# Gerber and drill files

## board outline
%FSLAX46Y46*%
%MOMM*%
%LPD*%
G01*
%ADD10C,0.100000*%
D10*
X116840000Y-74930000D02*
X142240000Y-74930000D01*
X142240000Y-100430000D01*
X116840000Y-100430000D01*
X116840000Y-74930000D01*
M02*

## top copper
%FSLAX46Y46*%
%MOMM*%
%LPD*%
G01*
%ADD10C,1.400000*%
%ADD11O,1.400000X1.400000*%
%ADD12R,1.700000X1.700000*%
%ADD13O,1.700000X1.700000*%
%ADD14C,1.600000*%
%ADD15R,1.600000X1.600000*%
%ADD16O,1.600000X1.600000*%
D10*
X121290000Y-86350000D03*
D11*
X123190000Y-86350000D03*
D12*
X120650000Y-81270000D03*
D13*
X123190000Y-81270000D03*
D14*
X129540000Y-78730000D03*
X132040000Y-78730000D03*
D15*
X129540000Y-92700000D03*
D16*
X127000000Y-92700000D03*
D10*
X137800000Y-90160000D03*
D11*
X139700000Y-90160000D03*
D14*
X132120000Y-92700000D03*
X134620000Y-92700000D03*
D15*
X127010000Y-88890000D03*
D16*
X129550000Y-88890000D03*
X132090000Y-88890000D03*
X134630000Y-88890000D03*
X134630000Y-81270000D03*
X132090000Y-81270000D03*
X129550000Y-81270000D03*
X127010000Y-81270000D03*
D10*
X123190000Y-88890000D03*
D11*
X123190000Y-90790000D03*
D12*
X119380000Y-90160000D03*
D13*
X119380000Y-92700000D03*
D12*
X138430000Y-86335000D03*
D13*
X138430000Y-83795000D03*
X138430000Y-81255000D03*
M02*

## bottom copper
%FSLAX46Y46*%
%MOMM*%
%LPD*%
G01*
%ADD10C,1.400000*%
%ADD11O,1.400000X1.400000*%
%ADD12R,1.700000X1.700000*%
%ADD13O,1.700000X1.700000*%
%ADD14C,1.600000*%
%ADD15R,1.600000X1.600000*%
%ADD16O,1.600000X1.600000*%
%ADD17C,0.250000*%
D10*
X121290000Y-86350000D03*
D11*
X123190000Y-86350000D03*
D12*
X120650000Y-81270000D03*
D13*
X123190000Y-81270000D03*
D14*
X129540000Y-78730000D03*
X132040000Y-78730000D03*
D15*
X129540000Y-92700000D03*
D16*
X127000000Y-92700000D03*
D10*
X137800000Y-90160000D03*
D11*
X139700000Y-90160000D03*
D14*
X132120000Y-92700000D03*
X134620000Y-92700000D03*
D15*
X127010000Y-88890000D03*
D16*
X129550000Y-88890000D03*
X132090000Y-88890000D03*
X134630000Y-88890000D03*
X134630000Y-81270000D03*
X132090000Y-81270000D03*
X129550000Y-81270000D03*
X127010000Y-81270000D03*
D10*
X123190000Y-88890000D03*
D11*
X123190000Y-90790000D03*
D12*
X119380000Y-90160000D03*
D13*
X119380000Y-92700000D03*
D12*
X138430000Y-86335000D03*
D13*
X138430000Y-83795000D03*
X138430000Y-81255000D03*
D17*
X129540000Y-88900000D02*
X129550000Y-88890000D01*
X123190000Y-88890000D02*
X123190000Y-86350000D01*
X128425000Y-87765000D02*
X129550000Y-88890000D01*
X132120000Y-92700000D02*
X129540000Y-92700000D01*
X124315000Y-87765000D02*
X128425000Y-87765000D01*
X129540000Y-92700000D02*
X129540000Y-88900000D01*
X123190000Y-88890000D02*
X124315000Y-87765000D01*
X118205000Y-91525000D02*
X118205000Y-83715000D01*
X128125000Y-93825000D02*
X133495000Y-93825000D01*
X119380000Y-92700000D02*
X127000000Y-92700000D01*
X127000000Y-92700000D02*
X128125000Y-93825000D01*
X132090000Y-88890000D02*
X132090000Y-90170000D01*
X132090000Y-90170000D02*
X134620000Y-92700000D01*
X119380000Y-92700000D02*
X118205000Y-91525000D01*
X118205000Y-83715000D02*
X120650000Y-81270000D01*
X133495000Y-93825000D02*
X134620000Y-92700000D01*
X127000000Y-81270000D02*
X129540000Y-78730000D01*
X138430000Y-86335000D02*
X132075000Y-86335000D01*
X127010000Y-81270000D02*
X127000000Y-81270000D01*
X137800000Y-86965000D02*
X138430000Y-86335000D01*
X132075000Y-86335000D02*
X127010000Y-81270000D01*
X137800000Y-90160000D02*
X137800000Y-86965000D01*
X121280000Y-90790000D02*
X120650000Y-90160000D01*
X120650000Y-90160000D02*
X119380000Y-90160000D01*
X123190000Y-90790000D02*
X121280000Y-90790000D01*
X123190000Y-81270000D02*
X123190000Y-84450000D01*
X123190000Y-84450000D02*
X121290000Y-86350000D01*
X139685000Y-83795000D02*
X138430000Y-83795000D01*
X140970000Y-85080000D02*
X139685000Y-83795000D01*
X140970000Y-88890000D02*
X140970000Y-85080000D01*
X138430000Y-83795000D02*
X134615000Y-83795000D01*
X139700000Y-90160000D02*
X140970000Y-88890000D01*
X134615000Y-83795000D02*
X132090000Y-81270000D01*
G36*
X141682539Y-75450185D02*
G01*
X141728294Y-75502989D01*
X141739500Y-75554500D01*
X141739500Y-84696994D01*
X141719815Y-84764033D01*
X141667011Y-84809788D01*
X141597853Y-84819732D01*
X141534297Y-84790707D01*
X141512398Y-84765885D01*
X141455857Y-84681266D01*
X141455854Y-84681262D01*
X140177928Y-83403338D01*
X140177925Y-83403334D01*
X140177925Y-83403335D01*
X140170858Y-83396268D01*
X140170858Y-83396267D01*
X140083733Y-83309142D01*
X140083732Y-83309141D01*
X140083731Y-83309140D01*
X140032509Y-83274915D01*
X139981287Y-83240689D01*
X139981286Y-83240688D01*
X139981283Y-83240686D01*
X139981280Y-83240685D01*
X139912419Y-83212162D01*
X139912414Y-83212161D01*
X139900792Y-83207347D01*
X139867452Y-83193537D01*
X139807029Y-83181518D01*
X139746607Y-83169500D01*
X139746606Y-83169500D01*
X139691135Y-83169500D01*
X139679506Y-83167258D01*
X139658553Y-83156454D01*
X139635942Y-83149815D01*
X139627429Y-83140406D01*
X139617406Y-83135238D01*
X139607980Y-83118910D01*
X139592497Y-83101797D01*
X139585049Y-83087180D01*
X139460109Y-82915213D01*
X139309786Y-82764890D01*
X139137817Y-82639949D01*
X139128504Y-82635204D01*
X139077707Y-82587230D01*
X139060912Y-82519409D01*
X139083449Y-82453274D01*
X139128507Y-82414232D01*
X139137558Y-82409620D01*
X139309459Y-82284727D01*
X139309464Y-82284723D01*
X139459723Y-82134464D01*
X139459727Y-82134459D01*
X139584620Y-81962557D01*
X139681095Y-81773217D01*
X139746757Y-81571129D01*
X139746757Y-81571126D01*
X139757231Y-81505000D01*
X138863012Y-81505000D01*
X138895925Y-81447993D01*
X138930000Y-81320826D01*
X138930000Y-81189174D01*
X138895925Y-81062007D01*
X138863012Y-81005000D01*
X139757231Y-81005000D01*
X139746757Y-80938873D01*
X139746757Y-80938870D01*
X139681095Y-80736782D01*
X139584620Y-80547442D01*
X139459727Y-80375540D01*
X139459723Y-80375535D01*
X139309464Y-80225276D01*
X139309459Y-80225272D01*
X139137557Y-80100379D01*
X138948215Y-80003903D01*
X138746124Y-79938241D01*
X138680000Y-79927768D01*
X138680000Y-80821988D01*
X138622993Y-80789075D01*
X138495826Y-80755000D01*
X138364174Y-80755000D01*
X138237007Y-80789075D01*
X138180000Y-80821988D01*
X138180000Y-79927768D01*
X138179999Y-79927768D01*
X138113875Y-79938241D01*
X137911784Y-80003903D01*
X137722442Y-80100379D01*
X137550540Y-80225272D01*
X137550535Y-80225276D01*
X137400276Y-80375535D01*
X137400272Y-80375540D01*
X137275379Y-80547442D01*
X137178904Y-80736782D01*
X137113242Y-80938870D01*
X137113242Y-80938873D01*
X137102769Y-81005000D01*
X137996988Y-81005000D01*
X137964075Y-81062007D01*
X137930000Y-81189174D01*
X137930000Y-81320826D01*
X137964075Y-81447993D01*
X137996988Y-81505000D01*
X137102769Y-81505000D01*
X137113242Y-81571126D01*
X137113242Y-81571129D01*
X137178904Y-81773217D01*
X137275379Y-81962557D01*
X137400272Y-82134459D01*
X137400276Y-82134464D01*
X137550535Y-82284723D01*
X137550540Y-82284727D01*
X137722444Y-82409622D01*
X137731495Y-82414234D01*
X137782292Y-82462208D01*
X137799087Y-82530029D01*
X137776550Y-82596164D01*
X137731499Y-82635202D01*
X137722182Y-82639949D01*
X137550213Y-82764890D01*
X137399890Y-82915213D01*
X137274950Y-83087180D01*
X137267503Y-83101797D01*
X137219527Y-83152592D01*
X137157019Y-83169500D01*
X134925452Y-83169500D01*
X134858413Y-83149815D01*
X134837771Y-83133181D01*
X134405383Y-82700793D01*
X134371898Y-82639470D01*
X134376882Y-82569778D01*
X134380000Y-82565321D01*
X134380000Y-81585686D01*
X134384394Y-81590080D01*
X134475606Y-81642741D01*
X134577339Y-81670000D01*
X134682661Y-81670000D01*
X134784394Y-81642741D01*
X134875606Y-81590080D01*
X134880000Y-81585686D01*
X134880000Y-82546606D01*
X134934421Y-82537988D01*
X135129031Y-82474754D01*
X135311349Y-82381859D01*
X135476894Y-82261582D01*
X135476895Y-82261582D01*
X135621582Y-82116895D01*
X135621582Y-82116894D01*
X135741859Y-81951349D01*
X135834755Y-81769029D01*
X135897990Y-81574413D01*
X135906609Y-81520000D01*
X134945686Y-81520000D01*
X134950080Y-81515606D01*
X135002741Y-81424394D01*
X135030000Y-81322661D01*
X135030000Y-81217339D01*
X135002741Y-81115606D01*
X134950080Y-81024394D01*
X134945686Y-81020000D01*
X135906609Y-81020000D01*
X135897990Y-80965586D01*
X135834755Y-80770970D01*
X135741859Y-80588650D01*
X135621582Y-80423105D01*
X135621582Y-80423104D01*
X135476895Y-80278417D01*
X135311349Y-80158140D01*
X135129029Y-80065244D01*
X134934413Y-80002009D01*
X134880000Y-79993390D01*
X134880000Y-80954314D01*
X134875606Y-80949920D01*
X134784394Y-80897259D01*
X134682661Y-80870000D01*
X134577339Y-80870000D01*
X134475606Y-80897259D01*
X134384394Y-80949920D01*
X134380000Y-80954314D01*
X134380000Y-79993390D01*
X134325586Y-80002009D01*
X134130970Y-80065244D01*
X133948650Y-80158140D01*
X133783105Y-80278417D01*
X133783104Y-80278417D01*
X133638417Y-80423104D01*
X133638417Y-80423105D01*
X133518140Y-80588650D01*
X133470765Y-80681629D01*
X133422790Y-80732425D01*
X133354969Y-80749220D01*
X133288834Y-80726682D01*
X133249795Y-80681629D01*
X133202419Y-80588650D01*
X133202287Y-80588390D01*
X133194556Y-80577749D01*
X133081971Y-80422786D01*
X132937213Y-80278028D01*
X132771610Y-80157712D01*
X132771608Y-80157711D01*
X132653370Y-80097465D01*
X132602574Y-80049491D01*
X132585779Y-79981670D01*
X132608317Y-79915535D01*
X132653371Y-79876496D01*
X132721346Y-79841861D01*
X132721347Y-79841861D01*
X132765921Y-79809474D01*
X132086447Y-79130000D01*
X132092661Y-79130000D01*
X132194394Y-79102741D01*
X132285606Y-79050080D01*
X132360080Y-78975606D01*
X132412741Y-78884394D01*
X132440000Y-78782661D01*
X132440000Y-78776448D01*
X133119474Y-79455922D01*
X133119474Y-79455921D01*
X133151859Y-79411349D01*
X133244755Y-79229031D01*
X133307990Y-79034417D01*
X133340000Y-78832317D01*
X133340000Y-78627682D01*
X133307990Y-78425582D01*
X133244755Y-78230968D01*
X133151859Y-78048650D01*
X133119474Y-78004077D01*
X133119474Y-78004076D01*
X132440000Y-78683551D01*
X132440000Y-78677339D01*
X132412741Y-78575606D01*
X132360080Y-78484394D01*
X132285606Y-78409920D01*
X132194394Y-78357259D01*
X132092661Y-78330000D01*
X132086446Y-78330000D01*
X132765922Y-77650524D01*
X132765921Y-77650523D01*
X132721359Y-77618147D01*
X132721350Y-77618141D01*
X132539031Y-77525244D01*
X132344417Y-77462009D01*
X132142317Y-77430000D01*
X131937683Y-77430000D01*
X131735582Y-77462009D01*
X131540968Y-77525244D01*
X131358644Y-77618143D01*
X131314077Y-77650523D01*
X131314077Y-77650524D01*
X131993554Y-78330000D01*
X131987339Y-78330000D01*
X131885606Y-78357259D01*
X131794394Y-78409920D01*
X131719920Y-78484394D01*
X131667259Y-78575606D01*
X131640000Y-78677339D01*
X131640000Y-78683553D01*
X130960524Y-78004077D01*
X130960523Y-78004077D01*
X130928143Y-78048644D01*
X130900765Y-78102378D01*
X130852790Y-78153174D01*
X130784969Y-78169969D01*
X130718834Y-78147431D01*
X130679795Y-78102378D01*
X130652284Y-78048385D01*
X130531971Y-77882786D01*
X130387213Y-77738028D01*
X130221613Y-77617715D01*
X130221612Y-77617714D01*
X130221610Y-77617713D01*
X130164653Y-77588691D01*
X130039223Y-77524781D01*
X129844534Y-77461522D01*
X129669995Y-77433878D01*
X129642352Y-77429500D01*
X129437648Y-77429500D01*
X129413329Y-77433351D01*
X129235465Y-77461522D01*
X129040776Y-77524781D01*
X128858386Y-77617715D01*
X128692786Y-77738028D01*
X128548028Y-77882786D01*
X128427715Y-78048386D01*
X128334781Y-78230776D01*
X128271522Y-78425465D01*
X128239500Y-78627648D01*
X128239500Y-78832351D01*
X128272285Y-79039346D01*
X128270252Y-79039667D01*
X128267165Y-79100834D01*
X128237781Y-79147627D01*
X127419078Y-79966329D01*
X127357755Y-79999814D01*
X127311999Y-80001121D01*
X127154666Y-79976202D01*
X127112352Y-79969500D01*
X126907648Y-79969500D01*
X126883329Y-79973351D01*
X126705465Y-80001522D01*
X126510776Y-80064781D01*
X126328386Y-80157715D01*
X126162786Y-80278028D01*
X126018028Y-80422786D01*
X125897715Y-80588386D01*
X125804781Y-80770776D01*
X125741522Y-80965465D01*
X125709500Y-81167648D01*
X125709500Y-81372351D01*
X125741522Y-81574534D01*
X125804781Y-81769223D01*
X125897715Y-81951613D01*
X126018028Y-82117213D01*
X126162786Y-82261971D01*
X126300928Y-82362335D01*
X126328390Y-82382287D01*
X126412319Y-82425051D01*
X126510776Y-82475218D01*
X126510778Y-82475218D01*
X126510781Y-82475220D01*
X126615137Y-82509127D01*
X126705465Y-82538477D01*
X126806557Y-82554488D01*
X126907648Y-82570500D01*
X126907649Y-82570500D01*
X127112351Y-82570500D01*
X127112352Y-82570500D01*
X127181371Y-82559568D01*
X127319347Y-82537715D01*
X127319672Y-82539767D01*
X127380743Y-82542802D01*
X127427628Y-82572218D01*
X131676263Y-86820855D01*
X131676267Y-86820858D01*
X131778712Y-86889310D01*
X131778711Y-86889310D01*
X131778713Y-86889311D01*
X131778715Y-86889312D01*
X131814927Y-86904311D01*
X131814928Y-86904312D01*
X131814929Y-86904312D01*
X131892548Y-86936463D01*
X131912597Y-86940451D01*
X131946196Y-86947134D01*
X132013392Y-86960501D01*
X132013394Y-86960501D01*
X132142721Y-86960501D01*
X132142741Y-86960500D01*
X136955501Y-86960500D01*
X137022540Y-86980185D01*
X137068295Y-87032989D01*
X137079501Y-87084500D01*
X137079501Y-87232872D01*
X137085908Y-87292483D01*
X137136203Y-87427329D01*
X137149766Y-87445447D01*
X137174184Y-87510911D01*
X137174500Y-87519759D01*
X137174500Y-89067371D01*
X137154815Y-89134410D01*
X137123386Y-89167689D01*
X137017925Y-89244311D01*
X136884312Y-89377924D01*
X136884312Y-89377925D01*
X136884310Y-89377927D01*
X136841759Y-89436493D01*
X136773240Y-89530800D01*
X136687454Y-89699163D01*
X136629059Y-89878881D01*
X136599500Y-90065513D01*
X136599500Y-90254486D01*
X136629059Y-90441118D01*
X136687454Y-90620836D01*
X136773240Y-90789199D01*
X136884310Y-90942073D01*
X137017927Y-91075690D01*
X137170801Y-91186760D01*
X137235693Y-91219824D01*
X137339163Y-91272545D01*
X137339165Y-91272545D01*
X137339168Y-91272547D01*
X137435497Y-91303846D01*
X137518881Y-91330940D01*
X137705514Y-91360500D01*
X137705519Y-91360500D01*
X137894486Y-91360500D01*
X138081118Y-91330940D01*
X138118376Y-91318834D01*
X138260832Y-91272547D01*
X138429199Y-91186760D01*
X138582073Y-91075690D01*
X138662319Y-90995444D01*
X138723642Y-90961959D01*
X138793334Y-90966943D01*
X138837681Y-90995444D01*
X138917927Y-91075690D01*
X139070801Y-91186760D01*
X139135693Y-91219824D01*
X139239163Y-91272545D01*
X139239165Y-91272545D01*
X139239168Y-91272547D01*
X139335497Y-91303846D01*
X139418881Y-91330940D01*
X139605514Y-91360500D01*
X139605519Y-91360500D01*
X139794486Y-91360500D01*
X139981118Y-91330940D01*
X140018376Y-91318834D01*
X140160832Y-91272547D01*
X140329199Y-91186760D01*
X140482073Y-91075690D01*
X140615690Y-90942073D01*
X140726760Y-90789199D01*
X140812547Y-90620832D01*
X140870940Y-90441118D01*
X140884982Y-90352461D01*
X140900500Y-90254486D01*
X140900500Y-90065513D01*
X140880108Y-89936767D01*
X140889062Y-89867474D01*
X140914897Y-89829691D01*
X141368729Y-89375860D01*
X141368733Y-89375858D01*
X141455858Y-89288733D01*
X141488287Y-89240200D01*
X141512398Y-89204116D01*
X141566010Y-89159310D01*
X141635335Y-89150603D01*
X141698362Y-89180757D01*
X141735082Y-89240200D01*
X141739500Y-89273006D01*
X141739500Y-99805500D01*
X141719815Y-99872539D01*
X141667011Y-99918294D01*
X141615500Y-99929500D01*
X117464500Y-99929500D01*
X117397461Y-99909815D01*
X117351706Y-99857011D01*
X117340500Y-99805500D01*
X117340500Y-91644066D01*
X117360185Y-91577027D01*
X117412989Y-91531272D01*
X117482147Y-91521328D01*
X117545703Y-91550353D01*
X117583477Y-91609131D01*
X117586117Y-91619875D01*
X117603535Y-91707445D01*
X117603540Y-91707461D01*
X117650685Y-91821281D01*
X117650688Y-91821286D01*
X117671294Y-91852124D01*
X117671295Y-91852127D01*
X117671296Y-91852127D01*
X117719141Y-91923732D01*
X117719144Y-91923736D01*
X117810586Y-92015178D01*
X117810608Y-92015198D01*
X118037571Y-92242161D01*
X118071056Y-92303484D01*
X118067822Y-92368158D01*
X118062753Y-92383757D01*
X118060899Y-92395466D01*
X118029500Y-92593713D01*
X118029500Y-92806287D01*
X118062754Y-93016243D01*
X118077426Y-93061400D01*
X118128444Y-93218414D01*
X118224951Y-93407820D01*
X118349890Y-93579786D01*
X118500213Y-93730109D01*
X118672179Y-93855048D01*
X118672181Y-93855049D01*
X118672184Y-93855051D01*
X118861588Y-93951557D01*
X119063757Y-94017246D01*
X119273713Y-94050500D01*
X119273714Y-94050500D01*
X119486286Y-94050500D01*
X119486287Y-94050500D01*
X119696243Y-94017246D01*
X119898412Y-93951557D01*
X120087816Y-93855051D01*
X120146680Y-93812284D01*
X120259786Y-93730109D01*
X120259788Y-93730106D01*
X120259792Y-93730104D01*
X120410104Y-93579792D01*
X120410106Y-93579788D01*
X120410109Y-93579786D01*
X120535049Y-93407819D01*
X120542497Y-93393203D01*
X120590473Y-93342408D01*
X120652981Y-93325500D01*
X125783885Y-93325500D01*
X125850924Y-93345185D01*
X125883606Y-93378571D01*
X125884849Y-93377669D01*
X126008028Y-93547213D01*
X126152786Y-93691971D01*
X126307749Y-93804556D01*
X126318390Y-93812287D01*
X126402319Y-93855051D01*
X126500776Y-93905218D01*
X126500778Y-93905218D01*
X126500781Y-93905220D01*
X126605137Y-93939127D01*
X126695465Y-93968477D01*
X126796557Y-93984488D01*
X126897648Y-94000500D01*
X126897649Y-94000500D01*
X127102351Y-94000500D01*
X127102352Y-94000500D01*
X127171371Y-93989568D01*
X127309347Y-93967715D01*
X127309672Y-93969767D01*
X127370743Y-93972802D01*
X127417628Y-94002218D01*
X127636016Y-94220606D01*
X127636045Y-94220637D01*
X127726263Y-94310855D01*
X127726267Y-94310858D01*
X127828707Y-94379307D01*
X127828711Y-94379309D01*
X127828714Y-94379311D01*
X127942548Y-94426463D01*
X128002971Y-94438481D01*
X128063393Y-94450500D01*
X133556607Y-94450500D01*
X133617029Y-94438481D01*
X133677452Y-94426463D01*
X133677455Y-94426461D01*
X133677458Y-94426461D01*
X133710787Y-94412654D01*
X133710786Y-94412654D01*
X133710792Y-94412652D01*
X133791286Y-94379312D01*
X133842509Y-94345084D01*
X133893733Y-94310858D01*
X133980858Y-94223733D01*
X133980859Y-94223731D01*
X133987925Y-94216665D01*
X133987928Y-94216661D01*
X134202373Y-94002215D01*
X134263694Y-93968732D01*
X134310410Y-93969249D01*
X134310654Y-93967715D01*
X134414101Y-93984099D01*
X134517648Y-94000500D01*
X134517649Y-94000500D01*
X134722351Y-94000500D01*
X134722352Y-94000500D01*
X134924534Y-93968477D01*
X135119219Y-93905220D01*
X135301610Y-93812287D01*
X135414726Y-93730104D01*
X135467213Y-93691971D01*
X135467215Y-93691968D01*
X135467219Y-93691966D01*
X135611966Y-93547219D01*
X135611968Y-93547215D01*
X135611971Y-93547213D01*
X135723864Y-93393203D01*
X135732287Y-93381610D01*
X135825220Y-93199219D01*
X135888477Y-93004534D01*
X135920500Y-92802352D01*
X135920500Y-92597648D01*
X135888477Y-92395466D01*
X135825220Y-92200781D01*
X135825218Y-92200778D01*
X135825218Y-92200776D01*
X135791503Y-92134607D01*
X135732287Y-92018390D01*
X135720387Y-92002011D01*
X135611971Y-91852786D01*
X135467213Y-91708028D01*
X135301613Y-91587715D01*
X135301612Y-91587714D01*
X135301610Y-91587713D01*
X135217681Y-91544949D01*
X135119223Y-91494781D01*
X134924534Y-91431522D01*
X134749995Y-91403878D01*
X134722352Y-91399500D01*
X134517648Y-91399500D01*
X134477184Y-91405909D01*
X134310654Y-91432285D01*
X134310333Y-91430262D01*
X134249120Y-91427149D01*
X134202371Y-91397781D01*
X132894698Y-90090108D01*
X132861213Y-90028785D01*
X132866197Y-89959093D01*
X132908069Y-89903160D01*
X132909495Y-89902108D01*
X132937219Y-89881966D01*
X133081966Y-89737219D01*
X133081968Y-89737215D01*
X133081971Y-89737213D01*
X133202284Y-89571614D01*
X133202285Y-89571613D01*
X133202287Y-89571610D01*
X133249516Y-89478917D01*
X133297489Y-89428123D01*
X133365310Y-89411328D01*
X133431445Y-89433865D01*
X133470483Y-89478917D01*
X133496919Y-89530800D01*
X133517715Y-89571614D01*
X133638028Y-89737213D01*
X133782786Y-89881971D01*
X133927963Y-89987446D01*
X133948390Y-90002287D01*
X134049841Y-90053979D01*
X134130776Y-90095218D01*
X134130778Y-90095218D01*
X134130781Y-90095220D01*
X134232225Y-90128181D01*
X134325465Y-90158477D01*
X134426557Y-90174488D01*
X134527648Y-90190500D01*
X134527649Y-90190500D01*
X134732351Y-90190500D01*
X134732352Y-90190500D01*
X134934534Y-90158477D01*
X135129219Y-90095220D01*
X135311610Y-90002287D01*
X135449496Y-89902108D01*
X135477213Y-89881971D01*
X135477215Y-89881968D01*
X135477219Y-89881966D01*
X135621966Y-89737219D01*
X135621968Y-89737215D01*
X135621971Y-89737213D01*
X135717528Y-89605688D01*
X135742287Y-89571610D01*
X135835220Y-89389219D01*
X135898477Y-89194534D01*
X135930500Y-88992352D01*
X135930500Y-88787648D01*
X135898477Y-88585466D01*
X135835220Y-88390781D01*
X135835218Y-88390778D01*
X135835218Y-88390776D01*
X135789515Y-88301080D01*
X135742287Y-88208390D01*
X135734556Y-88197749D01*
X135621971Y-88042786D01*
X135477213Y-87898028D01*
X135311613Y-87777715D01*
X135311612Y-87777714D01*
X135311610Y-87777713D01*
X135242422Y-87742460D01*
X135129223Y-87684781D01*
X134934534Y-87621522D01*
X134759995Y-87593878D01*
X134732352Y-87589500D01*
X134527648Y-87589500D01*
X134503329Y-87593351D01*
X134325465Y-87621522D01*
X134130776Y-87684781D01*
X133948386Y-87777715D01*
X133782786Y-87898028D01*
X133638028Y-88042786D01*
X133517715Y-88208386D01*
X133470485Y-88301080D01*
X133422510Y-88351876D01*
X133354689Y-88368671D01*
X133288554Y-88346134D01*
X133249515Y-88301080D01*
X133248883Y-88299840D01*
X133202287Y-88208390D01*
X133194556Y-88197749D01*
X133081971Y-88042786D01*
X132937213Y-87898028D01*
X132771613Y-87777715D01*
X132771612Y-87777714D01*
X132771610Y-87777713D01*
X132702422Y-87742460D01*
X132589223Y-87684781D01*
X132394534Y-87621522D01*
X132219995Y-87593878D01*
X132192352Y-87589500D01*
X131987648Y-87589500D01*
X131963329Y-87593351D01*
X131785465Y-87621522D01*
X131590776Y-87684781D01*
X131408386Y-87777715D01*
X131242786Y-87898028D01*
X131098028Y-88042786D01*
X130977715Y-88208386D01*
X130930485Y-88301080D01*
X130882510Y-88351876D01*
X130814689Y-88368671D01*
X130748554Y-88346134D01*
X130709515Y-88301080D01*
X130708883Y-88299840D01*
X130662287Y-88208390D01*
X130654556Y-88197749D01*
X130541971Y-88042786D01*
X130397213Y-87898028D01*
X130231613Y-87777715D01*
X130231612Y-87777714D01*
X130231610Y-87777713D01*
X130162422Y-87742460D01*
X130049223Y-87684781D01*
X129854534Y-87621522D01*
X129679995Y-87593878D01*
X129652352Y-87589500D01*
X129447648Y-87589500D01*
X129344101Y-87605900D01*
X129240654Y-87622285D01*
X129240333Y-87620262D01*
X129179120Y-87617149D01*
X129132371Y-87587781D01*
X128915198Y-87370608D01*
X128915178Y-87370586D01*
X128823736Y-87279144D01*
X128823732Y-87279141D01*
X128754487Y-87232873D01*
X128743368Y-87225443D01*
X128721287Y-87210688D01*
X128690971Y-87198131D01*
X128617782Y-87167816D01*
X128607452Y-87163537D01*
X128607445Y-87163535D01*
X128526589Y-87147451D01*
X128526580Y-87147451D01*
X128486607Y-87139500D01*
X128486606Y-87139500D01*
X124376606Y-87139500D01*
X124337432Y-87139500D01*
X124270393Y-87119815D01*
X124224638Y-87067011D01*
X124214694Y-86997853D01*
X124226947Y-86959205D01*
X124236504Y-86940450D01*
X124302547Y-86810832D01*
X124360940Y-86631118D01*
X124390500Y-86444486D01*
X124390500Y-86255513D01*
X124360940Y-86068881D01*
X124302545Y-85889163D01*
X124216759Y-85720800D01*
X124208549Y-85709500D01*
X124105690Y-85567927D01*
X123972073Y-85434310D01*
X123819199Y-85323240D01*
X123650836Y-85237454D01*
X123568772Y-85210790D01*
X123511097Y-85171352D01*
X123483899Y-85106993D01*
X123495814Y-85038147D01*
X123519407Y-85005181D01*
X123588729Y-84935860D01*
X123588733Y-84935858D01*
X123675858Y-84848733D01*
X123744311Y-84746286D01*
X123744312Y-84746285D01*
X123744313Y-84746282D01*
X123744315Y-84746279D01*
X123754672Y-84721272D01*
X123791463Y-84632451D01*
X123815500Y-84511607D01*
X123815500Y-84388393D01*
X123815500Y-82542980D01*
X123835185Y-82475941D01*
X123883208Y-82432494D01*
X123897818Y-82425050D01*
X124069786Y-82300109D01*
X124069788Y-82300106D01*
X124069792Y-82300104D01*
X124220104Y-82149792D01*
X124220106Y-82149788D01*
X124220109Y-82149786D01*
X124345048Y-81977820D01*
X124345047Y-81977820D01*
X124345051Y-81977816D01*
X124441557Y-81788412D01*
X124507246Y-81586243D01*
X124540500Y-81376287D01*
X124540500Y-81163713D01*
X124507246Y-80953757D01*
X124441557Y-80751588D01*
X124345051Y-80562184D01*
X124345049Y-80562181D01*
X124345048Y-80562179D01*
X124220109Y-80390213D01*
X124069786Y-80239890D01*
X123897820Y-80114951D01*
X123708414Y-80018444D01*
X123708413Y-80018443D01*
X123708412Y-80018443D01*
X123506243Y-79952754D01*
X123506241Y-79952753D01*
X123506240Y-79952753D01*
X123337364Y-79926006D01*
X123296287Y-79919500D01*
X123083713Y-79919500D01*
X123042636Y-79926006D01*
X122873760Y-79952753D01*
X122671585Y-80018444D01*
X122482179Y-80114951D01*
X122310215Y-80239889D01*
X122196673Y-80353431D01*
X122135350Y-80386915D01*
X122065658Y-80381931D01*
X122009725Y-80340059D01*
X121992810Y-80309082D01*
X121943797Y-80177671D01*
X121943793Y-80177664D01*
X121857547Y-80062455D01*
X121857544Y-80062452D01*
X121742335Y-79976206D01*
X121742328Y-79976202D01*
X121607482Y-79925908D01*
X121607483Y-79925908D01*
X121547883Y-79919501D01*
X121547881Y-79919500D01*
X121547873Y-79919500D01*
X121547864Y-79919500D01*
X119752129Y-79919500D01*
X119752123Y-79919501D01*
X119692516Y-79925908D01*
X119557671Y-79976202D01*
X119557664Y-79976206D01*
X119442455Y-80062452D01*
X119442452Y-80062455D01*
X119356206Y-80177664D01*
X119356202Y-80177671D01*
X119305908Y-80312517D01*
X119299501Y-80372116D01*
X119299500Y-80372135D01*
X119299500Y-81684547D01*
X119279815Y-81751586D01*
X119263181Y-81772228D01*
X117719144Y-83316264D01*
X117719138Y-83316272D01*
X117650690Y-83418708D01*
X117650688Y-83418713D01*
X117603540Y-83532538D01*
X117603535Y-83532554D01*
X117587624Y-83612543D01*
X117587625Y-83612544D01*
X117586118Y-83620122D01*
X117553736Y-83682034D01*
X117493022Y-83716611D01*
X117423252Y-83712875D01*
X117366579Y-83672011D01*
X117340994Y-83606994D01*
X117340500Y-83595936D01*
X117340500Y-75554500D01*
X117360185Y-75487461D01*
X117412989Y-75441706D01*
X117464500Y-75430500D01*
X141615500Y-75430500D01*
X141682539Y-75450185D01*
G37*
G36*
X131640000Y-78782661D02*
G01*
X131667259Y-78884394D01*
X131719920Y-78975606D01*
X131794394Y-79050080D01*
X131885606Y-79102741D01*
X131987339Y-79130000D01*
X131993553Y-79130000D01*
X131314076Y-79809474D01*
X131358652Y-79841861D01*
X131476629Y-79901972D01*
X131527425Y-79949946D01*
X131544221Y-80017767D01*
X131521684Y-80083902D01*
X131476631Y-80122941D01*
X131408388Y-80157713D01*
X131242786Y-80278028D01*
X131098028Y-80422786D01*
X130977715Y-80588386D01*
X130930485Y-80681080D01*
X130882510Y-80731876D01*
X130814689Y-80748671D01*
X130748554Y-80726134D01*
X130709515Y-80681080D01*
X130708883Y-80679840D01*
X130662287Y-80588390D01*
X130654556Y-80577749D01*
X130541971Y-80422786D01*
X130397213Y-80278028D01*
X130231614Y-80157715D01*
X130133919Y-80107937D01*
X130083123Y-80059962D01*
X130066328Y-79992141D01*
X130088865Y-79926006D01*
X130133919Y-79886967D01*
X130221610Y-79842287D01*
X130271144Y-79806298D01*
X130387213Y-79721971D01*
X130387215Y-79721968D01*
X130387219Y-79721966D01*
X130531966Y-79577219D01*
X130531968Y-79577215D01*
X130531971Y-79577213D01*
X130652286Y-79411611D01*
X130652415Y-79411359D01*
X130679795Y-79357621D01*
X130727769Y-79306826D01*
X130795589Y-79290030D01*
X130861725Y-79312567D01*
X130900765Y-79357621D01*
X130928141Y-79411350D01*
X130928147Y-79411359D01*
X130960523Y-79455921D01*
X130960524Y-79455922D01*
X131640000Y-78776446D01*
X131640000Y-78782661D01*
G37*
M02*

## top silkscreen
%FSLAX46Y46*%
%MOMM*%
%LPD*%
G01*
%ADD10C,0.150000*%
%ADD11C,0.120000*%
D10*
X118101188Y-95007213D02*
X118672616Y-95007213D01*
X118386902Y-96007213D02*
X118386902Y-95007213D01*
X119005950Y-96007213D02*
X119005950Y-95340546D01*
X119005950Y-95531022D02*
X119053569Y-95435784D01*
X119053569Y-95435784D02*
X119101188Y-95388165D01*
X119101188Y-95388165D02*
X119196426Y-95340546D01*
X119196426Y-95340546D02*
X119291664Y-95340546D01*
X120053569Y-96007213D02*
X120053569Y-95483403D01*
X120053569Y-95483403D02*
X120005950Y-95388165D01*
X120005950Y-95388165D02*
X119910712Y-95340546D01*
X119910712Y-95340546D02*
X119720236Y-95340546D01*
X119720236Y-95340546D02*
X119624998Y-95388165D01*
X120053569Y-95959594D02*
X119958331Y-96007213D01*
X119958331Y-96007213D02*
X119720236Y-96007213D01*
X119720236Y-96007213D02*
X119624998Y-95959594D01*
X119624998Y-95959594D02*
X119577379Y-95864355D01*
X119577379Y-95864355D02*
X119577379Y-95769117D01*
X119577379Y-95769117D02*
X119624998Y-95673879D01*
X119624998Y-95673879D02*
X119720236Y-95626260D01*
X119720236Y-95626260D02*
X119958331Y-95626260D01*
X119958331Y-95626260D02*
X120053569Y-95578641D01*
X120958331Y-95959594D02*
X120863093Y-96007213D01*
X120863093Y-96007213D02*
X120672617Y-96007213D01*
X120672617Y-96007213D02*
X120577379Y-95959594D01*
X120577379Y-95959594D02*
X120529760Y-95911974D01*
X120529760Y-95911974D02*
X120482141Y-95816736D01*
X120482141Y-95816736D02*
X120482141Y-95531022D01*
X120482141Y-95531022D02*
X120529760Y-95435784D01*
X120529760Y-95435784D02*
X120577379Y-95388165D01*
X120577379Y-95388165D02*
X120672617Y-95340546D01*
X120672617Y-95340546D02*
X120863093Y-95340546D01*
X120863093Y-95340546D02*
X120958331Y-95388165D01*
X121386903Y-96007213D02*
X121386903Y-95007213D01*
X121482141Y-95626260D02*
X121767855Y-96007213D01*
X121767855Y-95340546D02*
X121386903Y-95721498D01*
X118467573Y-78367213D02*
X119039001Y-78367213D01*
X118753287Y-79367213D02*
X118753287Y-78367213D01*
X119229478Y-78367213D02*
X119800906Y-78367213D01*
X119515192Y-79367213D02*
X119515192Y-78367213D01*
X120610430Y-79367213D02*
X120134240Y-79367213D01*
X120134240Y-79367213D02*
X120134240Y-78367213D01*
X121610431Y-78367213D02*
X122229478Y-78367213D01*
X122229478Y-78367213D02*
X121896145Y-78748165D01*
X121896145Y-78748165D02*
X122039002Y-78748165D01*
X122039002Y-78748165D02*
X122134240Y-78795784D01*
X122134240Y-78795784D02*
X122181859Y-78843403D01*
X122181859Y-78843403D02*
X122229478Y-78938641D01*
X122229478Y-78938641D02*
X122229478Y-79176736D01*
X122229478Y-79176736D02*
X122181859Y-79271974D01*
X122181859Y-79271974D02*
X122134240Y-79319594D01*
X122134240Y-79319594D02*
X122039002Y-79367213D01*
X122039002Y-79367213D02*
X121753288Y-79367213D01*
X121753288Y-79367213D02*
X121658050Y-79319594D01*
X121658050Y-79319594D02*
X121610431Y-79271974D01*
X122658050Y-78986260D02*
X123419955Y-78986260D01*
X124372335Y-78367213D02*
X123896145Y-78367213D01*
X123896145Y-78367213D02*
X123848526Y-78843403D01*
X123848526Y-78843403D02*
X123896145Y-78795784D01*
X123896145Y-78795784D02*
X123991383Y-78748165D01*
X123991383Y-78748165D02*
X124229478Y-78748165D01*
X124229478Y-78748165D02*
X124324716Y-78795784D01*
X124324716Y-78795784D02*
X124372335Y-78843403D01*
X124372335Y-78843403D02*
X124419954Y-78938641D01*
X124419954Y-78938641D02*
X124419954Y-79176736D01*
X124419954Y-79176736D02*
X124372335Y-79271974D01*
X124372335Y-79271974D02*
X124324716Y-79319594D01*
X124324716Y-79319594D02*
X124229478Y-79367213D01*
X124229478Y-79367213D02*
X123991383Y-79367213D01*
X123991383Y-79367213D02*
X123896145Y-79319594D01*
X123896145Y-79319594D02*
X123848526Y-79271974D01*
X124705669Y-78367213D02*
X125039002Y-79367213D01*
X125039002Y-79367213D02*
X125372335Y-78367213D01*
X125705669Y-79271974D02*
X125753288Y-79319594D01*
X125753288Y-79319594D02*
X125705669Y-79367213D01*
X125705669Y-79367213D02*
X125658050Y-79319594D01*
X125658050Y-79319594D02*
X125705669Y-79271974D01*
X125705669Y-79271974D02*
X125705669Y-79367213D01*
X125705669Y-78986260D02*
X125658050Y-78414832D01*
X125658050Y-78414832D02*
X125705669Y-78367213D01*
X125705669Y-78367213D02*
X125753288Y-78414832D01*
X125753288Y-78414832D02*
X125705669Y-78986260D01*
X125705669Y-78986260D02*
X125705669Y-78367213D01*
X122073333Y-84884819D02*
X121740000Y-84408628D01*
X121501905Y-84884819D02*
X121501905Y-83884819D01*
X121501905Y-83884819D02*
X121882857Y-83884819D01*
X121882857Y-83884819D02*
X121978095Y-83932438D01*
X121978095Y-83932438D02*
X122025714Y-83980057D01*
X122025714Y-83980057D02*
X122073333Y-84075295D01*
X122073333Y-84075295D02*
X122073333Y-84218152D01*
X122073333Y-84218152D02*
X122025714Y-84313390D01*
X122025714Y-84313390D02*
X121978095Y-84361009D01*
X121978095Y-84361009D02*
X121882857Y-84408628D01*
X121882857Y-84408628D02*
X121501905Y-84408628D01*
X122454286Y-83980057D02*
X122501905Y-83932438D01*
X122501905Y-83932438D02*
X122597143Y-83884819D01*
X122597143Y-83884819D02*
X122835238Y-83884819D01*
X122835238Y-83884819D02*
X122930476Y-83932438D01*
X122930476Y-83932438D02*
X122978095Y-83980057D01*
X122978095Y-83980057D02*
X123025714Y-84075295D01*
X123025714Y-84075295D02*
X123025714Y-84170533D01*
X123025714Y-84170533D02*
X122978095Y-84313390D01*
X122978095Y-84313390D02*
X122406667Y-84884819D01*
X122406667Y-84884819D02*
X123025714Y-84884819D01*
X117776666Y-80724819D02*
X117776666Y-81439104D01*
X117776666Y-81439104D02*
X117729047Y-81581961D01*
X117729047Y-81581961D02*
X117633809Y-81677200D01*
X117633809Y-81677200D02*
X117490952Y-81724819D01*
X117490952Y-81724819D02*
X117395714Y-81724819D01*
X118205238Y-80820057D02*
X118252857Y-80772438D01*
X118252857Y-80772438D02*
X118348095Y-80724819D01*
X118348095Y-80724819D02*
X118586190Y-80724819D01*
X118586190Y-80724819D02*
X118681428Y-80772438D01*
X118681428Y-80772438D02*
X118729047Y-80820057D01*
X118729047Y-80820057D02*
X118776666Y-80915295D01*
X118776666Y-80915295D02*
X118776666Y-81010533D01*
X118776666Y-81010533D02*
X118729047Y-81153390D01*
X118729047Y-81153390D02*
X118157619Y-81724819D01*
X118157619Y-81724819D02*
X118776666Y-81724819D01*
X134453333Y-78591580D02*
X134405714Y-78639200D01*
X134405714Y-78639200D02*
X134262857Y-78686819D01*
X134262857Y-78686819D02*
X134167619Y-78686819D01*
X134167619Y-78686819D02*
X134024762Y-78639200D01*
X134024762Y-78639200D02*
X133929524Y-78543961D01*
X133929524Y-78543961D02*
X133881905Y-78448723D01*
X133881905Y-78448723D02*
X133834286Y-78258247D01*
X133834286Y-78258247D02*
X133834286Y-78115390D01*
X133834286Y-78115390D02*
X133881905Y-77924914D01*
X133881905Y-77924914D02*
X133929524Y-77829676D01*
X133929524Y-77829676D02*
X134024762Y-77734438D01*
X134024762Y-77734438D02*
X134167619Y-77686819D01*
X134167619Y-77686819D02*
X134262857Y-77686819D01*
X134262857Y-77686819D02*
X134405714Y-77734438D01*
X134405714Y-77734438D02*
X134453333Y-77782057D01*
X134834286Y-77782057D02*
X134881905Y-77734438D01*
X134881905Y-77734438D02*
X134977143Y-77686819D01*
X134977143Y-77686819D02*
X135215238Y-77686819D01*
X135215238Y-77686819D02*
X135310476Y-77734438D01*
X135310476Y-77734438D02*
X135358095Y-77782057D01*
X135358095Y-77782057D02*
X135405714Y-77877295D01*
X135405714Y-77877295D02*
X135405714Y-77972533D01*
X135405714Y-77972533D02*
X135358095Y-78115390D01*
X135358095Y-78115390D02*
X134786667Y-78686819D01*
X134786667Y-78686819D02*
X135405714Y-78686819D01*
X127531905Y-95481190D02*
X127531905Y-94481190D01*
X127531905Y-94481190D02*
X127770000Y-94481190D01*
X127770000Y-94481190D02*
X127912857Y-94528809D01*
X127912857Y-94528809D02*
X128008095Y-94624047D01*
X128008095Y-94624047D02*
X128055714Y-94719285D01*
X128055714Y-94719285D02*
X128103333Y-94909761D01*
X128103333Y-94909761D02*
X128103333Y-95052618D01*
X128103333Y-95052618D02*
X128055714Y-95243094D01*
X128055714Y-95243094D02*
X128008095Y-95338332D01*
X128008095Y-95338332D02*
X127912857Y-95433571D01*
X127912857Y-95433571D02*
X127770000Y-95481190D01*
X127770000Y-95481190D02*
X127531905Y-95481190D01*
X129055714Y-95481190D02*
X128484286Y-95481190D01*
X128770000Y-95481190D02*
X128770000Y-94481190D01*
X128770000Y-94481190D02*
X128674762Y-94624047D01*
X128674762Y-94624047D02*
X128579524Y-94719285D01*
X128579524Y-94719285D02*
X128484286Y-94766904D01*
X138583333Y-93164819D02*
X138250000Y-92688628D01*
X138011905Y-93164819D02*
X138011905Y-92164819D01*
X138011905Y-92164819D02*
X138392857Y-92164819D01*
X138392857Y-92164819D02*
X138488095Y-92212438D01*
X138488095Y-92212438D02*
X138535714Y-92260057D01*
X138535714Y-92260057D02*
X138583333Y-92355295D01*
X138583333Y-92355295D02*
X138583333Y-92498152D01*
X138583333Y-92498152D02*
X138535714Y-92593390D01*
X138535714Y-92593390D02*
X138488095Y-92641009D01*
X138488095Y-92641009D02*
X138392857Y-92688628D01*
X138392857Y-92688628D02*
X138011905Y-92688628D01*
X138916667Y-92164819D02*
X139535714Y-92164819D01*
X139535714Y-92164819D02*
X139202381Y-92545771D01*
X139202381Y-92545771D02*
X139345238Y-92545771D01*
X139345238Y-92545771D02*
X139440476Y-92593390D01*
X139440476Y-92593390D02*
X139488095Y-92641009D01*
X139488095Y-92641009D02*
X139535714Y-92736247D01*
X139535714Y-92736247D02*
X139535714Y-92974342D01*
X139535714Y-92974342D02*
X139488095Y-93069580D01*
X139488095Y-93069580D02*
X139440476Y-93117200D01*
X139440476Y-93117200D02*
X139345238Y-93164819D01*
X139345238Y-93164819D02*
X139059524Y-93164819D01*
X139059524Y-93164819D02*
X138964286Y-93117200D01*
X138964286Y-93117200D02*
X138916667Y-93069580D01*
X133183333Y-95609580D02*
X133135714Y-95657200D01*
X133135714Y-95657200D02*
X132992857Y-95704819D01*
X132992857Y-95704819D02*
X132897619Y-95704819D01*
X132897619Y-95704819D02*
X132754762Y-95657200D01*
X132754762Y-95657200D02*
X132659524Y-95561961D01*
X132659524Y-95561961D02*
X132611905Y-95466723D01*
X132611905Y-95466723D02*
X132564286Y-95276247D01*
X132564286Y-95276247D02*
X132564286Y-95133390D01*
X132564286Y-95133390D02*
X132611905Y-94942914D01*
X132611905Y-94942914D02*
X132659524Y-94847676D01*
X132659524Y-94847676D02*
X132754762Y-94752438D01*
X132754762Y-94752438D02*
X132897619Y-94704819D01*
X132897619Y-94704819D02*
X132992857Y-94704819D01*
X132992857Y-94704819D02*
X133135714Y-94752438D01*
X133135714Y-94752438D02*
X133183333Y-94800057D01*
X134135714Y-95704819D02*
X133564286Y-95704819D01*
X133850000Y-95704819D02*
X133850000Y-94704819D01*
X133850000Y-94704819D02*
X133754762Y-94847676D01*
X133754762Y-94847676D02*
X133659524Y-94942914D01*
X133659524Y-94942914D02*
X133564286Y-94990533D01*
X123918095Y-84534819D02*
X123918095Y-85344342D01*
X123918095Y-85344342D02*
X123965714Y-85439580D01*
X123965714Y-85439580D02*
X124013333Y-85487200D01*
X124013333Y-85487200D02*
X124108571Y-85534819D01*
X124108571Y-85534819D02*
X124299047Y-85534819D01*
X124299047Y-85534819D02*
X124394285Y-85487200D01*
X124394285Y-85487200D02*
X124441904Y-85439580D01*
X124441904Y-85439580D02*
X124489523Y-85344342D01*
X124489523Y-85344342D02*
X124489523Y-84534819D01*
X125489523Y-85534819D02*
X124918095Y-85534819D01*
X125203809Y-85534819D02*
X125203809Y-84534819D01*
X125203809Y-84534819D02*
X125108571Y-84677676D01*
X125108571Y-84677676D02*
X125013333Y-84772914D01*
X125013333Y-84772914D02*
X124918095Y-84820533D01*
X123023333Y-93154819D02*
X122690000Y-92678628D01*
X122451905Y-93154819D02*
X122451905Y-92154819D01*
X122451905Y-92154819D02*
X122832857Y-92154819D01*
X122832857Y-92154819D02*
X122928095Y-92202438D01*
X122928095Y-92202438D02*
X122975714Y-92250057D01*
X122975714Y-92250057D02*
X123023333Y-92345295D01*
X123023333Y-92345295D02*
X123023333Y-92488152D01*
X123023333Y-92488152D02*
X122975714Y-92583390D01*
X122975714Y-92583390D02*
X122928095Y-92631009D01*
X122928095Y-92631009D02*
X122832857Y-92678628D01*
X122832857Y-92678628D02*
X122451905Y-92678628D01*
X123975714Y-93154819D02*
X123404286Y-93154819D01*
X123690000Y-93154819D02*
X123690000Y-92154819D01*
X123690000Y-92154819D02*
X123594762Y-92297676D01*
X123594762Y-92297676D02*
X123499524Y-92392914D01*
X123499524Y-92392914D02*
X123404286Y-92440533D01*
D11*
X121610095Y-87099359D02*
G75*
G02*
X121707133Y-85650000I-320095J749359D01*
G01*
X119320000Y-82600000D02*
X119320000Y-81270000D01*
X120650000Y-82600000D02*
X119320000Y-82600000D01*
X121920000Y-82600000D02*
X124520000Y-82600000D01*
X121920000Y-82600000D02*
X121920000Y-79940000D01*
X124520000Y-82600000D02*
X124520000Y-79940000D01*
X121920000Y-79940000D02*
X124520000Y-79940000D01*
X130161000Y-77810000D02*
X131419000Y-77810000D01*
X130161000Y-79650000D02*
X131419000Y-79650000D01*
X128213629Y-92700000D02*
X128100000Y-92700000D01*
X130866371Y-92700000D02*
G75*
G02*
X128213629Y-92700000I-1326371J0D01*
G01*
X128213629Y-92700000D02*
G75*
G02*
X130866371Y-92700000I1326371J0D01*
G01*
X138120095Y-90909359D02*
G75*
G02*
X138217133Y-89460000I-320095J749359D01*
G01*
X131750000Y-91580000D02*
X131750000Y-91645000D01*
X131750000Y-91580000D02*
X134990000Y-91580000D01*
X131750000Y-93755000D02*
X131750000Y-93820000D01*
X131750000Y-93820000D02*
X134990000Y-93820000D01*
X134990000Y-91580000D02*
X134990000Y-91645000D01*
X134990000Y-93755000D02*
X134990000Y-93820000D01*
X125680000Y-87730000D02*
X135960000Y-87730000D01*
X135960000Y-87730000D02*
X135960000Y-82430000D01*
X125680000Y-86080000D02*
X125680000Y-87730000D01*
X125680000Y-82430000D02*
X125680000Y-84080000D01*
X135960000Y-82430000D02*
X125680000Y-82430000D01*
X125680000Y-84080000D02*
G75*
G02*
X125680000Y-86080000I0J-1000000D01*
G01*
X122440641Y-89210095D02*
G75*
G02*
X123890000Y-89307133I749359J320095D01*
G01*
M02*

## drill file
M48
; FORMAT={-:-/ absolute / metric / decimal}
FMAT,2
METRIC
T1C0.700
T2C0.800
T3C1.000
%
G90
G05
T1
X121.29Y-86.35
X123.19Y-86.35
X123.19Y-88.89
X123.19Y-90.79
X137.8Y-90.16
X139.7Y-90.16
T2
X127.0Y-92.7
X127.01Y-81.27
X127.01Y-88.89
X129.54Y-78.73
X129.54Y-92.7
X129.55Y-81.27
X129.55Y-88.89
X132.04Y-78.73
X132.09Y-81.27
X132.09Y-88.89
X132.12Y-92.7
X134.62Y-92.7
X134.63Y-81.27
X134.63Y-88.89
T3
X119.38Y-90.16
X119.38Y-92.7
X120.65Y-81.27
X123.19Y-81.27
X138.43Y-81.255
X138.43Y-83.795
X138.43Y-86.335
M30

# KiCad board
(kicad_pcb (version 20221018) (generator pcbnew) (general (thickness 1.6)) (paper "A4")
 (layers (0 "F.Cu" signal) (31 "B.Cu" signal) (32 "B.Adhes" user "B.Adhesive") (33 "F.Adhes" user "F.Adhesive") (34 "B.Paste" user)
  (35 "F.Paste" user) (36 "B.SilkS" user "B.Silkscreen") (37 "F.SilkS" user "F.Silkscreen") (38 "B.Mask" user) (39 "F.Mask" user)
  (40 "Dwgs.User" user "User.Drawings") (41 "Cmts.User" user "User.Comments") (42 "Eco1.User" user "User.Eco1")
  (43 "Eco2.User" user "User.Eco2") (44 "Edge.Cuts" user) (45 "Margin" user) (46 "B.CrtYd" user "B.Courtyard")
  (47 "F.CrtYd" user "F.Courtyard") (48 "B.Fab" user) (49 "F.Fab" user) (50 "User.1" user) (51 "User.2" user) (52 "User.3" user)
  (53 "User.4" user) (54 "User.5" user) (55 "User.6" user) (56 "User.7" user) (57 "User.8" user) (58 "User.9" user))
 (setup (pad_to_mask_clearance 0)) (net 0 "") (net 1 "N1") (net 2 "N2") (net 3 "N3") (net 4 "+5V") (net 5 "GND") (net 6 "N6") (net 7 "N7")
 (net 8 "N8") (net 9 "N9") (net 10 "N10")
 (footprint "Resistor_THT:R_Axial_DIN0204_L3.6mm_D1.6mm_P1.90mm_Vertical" (layer "F.Cu") (at 121.29 86.35)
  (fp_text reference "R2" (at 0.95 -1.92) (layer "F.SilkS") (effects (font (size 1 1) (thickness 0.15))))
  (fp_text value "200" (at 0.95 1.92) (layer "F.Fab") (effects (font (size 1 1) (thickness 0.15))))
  (fp_arc (start 0.320095 0.749359) (mid -0.813042 -0.054435) (end 0.417133 -0.7) (stroke (width 0.12) (type solid)) (layer "F.SilkS"))
  (pad "1" thru_hole circle (at 0 0) (size 1.4 1.4) (drill 0.7) (layers "*.Cu" "*.Mask") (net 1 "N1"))
  (pad "2" thru_hole oval (at 1.9 0) (size 1.4 1.4) (drill 0.7) (layers "*.Cu" "*.Mask") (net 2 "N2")))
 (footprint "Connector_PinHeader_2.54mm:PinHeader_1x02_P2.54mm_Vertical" (layer "F.Cu") (at 120.65 81.27 90)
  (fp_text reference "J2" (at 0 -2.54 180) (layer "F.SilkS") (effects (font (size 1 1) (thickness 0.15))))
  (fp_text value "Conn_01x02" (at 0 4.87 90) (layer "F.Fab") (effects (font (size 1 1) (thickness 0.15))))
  (fp_line (start -1.33 -1.33) (end 0 -1.33) (stroke (width 0.12) (type solid)) (layer "F.SilkS"))
  (fp_line (start -1.33 0) (end -1.33 -1.33) (stroke (width 0.12) (type solid)) (layer "F.SilkS"))
  (fp_line (start -1.33 1.27) (end -1.33 3.87) (stroke (width 0.12) (type solid)) (layer "F.SilkS"))
  (fp_line (start -1.33 1.27) (end 1.33 1.27) (stroke (width 0.12) (type solid)) (layer "F.SilkS"))
  (fp_line (start -1.33 3.87) (end 1.33 3.87) (stroke (width 0.12) (type solid)) (layer "F.SilkS"))
  (fp_line (start 1.33 1.27) (end 1.33 3.87) (stroke (width 0.12) (type solid)) (layer "F.SilkS"))
  (pad "1" thru_hole rect (at 0 0 90) (size 1.7 1.7) (drill 1) (layers "*.Cu" "*.Mask") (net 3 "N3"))
  (pad "2" thru_hole oval (at 0 2.54 90) (size 1.7 1.7) (drill 1) (layers "*.Cu" "*.Mask") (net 1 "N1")))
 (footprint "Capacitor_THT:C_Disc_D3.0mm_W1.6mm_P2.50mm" (layer "F.Cu") (at 129.54 78.73)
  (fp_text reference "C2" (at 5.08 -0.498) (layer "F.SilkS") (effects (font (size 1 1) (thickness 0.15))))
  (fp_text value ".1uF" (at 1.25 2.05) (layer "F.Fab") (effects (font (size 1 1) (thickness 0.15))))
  (fp_line (start 0.621 -0.92) (end 1.879 -0.92) (stroke (width 0.12) (type solid)) (layer "F.SilkS"))
  (fp_line (start 0.621 0.92) (end 1.879 0.92) (stroke (width 0.12) (type solid)) (layer "F.SilkS"))
  (pad "1" thru_hole circle (at 0 0) (size 1.6 1.6) (drill 0.8) (layers "*.Cu" "*.Mask") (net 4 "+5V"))
  (pad "2" thru_hole circle (at 2.5 0) (size 1.6 1.6) (drill 0.8) (layers "*.Cu" "*.Mask") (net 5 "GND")))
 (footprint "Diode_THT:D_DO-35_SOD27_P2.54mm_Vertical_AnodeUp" (layer "F.Cu") (at 129.54 92.7 180)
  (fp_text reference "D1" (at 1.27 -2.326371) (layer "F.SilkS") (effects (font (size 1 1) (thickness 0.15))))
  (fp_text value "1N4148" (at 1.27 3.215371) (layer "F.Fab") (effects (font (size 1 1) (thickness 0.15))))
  (fp_line (start 1.326371 0) (end 1.44 0) (stroke (width 0.12) (type solid)) (layer "F.SilkS"))
  (fp_circle (center 0 0) (end 1.326371 0) (stroke (width 0.12) (type solid)) (fill none) (layer "F.SilkS"))
  (pad "1" thru_hole rect (at 0 0 180) (size 1.6 1.6) (drill 0.8) (layers "*.Cu" "*.Mask") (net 2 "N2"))
  (pad "2" thru_hole oval (at 2.54 0 180) (size 1.6 1.6) (drill 0.8) (layers "*.Cu" "*.Mask") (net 3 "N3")))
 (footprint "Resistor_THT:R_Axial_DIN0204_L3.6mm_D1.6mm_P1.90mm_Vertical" (layer "F.Cu") (at 137.8 90.16)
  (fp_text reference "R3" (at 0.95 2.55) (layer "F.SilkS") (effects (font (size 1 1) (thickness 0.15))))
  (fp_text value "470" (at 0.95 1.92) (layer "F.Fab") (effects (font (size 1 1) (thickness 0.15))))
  (fp_arc (start 0.320095 0.749359) (mid -0.813042 -0.054435) (end 0.417133 -0.7) (stroke (width 0.12) (type solid)) (layer "F.SilkS"))
  (pad "1" thru_hole circle (at 0 0) (size 1.4 1.4) (drill 0.7) (layers "*.Cu" "*.Mask") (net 4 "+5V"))
  (pad "2" thru_hole oval (at 1.9 0) (size 1.4 1.4) (drill 0.7) (layers "*.Cu" "*.Mask") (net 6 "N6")))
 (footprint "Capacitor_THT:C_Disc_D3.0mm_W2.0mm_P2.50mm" (layer "F.Cu") (at 132.12 92.7)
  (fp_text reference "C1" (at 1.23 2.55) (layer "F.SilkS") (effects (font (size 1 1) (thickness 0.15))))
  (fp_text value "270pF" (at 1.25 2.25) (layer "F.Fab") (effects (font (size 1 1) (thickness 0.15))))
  (fp_line (start -0.37 -1.12) (end -0.37 -1.055) (stroke (width 0.12) (type solid)) (layer "F.SilkS"))
  (fp_line (start -0.37 -1.12) (end 2.87 -1.12) (stroke (width 0.12) (type solid)) (layer "F.SilkS"))
  (fp_line (start -0.37 1.055) (end -0.37 1.12) (stroke (width 0.12) (type solid)) (layer "F.SilkS"))
  (fp_line (start -0.37 1.12) (end 2.87 1.12) (stroke (width 0.12) (type solid)) (layer "F.SilkS"))
  (fp_line (start 2.87 -1.12) (end 2.87 -1.055) (stroke (width 0.12) (type solid)) (layer "F.SilkS"))
  (fp_line (start 2.87 1.055) (end 2.87 1.12) (stroke (width 0.12) (type solid)) (layer "F.SilkS"))
  (pad "1" thru_hole circle (at 0 0) (size 1.6 1.6) (drill 0.8) (layers "*.Cu" "*.Mask") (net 2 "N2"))
  (pad "2" thru_hole circle (at 2.5 0) (size 1.6 1.6) (drill 0.8) (layers "*.Cu" "*.Mask") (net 3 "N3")))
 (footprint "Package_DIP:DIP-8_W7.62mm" (layer "F.Cu") (at 127.01 88.89 90)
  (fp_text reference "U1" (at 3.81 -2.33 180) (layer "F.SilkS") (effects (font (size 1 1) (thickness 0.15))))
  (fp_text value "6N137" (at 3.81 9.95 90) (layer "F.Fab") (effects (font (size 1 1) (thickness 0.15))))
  (fp_line (start 1.16 -1.33) (end 1.16 8.95) (stroke (width 0.12) (type solid)) (layer "F.SilkS"))
  (fp_line (start 1.16 8.95) (end 6.46 8.95) (stroke (width 0.12) (type solid)) (layer "F.SilkS"))
  (fp_line (start 2.81 -1.33) (end 1.16 -1.33) (stroke (width 0.12) (type solid)) (layer "F.SilkS"))
  (fp_line (start 6.46 -1.33) (end 4.81 -1.33) (stroke (width 0.12) (type solid)) (layer "F.SilkS"))
  (fp_line (start 6.46 8.95) (end 6.46 -1.33) (stroke (width 0.12) (type solid)) (layer "F.SilkS"))
  (fp_arc (start 4.81 -1.33) (mid 3.81 -0.33) (end 2.81 -1.33) (stroke (width 0.12) (type solid)) (layer "F.SilkS"))
  (pad "1" thru_hole rect (at 0 0 90) (size 1.6 1.6) (drill 0.8) (layers "*.Cu" "*.Mask") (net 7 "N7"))
  (pad "2" thru_hole oval (at 0 2.54 90) (size 1.6 1.6) (drill 0.8) (layers "*.Cu" "*.Mask") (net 2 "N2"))
  (pad "3" thru_hole oval (at 0 5.08 90) (size 1.6 1.6) (drill 0.8) (layers "*.Cu" "*.Mask") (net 3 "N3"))
  (pad "4" thru_hole oval (at 0 7.62 90) (size 1.6 1.6) (drill 0.8) (layers "*.Cu" "*.Mask") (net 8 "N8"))
  (pad "5" thru_hole oval (at 7.62 7.62 90) (size 1.6 1.6) (drill 0.8) (layers "*.Cu" "*.Mask") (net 5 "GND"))
  (pad "6" thru_hole oval (at 7.62 5.08 90) (size 1.6 1.6) (drill 0.8) (layers "*.Cu" "*.Mask") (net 6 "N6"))
  (pad "7" thru_hole oval (at 7.62 2.54 90) (size 1.6 1.6) (drill 0.8) (layers "*.Cu" "*.Mask") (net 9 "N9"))
  (pad "8" thru_hole oval (at 7.62 0 90) (size 1.6 1.6) (drill 0.8) (layers "*.Cu" "*.Mask") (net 4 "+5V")))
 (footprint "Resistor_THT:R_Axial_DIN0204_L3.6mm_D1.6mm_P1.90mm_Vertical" (layer "F.Cu") (at 123.19 88.89 -90)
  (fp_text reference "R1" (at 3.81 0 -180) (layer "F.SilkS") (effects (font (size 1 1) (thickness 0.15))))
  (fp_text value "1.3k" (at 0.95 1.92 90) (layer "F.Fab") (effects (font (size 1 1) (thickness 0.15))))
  (fp_arc (start 0.320095 0.749359) (mid -0.813042 -0.054435) (end 0.417133 -0.7) (stroke (width 0.12) (type solid)) (layer "F.SilkS"))
  (pad "1" thru_hole circle (at 0 0 270) (size 1.4 1.4) (drill 0.7) (layers "*.Cu" "*.Mask") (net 2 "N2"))
  (pad "2" thru_hole oval (at 1.9 0 270) (size 1.4 1.4) (drill 0.7) (layers "*.Cu" "*.Mask") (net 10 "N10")))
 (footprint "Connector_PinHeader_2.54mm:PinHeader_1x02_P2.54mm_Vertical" (layer "B.Cu") (at 119.38 90.16 180)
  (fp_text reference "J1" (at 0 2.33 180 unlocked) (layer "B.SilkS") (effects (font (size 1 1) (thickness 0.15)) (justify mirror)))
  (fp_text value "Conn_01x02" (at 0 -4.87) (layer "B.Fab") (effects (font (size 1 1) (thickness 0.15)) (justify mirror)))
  (pad "1" thru_hole rect (at 0 0 180) (size 1.7 1.7) (drill 1) (layers "*.Cu" "*.Mask") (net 10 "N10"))
  (pad "2" thru_hole oval (at 0 -2.54 180) (size 1.7 1.7) (drill 1) (layers "*.Cu" "*.Mask") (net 3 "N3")))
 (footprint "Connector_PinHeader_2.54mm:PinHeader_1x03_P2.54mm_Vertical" (layer "B.Cu") (at 138.43 86.335)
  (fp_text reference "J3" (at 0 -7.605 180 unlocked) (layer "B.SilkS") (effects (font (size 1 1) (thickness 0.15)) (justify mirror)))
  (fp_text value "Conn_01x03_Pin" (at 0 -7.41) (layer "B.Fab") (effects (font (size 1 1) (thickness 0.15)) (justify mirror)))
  (pad "1" thru_hole rect (at 0 0) (size 1.7 1.7) (drill 1) (layers "*.Cu" "*.Mask") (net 4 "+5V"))
  (pad "2" thru_hole oval (at 0 -2.54) (size 1.7 1.7) (drill 1) (layers "*.Cu" "*.Mask") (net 6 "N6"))
  (pad "3" thru_hole oval (at 0 -5.08) (size 1.7 1.7) (drill 1) (layers "*.Cu" "*.Mask") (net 5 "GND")))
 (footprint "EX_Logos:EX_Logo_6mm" (layer "B.Cu") (at 137.668 97.028)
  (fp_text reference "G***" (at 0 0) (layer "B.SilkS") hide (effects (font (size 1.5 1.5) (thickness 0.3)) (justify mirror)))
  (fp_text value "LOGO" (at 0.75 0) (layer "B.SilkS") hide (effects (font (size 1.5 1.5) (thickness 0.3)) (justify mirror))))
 (gr_rect (start 116.84 74.93) (end 142.24 100.43) (stroke (width 0.1) (type default)) (fill none) (layer "Edge.Cuts"))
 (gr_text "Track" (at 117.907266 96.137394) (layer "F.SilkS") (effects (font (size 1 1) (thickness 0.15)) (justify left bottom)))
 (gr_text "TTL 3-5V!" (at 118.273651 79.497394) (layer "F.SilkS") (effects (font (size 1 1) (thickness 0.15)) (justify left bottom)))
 (segment (start 129.54 88.9) (end 129.55 88.89) (width 0.25) (layer "B.Cu") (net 2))
 (segment (start 123.19 88.89) (end 123.19 86.35) (width 0.25) (layer "B.Cu") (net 2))
 (segment (start 128.425 87.765) (end 129.55 88.89) (width 0.25) (layer "B.Cu") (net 2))
 (segment (start 132.12 92.7) (end 129.54 92.7) (width 0.25) (layer "B.Cu") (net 2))
 (segment (start 124.315 87.765) (end 128.425 87.765) (width 0.25) (layer "B.Cu") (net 2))
 (segment (start 129.54 92.7) (end 129.54 88.9) (width 0.25) (layer "B.Cu") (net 2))
 (segment (start 123.19 88.89) (end 124.315 87.765) (width 0.25) (layer "B.Cu") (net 2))
 (segment (start 118.205 91.525) (end 118.205 83.715) (width 0.25) (layer "B.Cu") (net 3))
 (segment (start 128.125 93.825) (end 133.495 93.825) (width 0.25) (layer "B.Cu") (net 3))
 (segment (start 119.38 92.7) (end 127 92.7) (width 0.25) (layer "B.Cu") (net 3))
 (segment (start 127 92.7) (end 128.125 93.825) (width 0.25) (layer "B.Cu") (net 3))
 (segment (start 132.09 88.89) (end 132.09 90.17) (width 0.25) (layer "B.Cu") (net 3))
 (segment (start 132.09 90.17) (end 134.62 92.7) (width 0.25) (layer "B.Cu") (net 3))
 (segment (start 119.38 92.7) (end 118.205 91.525) (width 0.25) (layer "B.Cu") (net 3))
 (segment (start 118.205 83.715) (end 120.65 81.27) (width 0.25) (layer "B.Cu") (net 3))
 (segment (start 133.495 93.825) (end 134.62 92.7) (width 0.25) (layer "B.Cu") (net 3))
 (segment (start 127 81.27) (end 129.54 78.73) (width 0.25) (layer "B.Cu") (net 4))
 (segment (start 138.43 86.335) (end 132.075 86.335) (width 0.25) (layer "B.Cu") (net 4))
 (segment (start 127.01 81.27) (end 127 81.27) (width 0.25) (layer "B.Cu") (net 4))
 (segment (start 137.8 86.965) (end 138.43 86.335) (width 0.25) (layer "B.Cu") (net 4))
 (segment (start 132.075 86.335) (end 127.01 81.27) (width 0.25) (layer "B.Cu") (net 4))
 (segment (start 137.8 90.16) (end 137.8 86.965) (width 0.25) (layer "B.Cu") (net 4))
 (segment (start 121.28 90.79) (end 120.65 90.16) (width 0.25) (layer "B.Cu") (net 10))
 (segment (start 120.65 90.16) (end 119.38 90.16) (width 0.25) (layer "B.Cu") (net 10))
 (segment (start 123.19 90.79) (end 121.28 90.79) (width 0.25) (layer "B.Cu") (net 10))
 (segment (start 123.19 81.27) (end 123.19 84.45) (width 0.25) (layer "B.Cu") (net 1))
 (segment (start 123.19 84.45) (end 121.29 86.35) (width 0.25) (layer "B.Cu") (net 1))
 (segment (start 139.685 83.795) (end 138.43 83.795) (width 0.25) (layer "B.Cu") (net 6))
 (segment (start 140.97 85.08) (end 139.685 83.795) (width 0.25) (layer "B.Cu") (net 6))
 (segment (start 140.97 88.89) (end 140.97 85.08) (width 0.25) (layer "B.Cu") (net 6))
 (segment (start 138.43 83.795) (end 134.615 83.795) (width 0.25) (layer "B.Cu") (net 6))
 (segment (start 139.7 90.16) (end 140.97 88.89) (width 0.25) (layer "B.Cu") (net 6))
 (segment (start 134.615 83.795) (end 132.09 81.27) (width 0.25) (layer "B.Cu") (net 6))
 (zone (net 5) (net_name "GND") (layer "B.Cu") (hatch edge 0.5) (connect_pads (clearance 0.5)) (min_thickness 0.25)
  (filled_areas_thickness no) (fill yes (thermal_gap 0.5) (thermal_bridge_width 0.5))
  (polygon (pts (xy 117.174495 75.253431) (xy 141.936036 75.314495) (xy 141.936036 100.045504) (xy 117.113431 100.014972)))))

